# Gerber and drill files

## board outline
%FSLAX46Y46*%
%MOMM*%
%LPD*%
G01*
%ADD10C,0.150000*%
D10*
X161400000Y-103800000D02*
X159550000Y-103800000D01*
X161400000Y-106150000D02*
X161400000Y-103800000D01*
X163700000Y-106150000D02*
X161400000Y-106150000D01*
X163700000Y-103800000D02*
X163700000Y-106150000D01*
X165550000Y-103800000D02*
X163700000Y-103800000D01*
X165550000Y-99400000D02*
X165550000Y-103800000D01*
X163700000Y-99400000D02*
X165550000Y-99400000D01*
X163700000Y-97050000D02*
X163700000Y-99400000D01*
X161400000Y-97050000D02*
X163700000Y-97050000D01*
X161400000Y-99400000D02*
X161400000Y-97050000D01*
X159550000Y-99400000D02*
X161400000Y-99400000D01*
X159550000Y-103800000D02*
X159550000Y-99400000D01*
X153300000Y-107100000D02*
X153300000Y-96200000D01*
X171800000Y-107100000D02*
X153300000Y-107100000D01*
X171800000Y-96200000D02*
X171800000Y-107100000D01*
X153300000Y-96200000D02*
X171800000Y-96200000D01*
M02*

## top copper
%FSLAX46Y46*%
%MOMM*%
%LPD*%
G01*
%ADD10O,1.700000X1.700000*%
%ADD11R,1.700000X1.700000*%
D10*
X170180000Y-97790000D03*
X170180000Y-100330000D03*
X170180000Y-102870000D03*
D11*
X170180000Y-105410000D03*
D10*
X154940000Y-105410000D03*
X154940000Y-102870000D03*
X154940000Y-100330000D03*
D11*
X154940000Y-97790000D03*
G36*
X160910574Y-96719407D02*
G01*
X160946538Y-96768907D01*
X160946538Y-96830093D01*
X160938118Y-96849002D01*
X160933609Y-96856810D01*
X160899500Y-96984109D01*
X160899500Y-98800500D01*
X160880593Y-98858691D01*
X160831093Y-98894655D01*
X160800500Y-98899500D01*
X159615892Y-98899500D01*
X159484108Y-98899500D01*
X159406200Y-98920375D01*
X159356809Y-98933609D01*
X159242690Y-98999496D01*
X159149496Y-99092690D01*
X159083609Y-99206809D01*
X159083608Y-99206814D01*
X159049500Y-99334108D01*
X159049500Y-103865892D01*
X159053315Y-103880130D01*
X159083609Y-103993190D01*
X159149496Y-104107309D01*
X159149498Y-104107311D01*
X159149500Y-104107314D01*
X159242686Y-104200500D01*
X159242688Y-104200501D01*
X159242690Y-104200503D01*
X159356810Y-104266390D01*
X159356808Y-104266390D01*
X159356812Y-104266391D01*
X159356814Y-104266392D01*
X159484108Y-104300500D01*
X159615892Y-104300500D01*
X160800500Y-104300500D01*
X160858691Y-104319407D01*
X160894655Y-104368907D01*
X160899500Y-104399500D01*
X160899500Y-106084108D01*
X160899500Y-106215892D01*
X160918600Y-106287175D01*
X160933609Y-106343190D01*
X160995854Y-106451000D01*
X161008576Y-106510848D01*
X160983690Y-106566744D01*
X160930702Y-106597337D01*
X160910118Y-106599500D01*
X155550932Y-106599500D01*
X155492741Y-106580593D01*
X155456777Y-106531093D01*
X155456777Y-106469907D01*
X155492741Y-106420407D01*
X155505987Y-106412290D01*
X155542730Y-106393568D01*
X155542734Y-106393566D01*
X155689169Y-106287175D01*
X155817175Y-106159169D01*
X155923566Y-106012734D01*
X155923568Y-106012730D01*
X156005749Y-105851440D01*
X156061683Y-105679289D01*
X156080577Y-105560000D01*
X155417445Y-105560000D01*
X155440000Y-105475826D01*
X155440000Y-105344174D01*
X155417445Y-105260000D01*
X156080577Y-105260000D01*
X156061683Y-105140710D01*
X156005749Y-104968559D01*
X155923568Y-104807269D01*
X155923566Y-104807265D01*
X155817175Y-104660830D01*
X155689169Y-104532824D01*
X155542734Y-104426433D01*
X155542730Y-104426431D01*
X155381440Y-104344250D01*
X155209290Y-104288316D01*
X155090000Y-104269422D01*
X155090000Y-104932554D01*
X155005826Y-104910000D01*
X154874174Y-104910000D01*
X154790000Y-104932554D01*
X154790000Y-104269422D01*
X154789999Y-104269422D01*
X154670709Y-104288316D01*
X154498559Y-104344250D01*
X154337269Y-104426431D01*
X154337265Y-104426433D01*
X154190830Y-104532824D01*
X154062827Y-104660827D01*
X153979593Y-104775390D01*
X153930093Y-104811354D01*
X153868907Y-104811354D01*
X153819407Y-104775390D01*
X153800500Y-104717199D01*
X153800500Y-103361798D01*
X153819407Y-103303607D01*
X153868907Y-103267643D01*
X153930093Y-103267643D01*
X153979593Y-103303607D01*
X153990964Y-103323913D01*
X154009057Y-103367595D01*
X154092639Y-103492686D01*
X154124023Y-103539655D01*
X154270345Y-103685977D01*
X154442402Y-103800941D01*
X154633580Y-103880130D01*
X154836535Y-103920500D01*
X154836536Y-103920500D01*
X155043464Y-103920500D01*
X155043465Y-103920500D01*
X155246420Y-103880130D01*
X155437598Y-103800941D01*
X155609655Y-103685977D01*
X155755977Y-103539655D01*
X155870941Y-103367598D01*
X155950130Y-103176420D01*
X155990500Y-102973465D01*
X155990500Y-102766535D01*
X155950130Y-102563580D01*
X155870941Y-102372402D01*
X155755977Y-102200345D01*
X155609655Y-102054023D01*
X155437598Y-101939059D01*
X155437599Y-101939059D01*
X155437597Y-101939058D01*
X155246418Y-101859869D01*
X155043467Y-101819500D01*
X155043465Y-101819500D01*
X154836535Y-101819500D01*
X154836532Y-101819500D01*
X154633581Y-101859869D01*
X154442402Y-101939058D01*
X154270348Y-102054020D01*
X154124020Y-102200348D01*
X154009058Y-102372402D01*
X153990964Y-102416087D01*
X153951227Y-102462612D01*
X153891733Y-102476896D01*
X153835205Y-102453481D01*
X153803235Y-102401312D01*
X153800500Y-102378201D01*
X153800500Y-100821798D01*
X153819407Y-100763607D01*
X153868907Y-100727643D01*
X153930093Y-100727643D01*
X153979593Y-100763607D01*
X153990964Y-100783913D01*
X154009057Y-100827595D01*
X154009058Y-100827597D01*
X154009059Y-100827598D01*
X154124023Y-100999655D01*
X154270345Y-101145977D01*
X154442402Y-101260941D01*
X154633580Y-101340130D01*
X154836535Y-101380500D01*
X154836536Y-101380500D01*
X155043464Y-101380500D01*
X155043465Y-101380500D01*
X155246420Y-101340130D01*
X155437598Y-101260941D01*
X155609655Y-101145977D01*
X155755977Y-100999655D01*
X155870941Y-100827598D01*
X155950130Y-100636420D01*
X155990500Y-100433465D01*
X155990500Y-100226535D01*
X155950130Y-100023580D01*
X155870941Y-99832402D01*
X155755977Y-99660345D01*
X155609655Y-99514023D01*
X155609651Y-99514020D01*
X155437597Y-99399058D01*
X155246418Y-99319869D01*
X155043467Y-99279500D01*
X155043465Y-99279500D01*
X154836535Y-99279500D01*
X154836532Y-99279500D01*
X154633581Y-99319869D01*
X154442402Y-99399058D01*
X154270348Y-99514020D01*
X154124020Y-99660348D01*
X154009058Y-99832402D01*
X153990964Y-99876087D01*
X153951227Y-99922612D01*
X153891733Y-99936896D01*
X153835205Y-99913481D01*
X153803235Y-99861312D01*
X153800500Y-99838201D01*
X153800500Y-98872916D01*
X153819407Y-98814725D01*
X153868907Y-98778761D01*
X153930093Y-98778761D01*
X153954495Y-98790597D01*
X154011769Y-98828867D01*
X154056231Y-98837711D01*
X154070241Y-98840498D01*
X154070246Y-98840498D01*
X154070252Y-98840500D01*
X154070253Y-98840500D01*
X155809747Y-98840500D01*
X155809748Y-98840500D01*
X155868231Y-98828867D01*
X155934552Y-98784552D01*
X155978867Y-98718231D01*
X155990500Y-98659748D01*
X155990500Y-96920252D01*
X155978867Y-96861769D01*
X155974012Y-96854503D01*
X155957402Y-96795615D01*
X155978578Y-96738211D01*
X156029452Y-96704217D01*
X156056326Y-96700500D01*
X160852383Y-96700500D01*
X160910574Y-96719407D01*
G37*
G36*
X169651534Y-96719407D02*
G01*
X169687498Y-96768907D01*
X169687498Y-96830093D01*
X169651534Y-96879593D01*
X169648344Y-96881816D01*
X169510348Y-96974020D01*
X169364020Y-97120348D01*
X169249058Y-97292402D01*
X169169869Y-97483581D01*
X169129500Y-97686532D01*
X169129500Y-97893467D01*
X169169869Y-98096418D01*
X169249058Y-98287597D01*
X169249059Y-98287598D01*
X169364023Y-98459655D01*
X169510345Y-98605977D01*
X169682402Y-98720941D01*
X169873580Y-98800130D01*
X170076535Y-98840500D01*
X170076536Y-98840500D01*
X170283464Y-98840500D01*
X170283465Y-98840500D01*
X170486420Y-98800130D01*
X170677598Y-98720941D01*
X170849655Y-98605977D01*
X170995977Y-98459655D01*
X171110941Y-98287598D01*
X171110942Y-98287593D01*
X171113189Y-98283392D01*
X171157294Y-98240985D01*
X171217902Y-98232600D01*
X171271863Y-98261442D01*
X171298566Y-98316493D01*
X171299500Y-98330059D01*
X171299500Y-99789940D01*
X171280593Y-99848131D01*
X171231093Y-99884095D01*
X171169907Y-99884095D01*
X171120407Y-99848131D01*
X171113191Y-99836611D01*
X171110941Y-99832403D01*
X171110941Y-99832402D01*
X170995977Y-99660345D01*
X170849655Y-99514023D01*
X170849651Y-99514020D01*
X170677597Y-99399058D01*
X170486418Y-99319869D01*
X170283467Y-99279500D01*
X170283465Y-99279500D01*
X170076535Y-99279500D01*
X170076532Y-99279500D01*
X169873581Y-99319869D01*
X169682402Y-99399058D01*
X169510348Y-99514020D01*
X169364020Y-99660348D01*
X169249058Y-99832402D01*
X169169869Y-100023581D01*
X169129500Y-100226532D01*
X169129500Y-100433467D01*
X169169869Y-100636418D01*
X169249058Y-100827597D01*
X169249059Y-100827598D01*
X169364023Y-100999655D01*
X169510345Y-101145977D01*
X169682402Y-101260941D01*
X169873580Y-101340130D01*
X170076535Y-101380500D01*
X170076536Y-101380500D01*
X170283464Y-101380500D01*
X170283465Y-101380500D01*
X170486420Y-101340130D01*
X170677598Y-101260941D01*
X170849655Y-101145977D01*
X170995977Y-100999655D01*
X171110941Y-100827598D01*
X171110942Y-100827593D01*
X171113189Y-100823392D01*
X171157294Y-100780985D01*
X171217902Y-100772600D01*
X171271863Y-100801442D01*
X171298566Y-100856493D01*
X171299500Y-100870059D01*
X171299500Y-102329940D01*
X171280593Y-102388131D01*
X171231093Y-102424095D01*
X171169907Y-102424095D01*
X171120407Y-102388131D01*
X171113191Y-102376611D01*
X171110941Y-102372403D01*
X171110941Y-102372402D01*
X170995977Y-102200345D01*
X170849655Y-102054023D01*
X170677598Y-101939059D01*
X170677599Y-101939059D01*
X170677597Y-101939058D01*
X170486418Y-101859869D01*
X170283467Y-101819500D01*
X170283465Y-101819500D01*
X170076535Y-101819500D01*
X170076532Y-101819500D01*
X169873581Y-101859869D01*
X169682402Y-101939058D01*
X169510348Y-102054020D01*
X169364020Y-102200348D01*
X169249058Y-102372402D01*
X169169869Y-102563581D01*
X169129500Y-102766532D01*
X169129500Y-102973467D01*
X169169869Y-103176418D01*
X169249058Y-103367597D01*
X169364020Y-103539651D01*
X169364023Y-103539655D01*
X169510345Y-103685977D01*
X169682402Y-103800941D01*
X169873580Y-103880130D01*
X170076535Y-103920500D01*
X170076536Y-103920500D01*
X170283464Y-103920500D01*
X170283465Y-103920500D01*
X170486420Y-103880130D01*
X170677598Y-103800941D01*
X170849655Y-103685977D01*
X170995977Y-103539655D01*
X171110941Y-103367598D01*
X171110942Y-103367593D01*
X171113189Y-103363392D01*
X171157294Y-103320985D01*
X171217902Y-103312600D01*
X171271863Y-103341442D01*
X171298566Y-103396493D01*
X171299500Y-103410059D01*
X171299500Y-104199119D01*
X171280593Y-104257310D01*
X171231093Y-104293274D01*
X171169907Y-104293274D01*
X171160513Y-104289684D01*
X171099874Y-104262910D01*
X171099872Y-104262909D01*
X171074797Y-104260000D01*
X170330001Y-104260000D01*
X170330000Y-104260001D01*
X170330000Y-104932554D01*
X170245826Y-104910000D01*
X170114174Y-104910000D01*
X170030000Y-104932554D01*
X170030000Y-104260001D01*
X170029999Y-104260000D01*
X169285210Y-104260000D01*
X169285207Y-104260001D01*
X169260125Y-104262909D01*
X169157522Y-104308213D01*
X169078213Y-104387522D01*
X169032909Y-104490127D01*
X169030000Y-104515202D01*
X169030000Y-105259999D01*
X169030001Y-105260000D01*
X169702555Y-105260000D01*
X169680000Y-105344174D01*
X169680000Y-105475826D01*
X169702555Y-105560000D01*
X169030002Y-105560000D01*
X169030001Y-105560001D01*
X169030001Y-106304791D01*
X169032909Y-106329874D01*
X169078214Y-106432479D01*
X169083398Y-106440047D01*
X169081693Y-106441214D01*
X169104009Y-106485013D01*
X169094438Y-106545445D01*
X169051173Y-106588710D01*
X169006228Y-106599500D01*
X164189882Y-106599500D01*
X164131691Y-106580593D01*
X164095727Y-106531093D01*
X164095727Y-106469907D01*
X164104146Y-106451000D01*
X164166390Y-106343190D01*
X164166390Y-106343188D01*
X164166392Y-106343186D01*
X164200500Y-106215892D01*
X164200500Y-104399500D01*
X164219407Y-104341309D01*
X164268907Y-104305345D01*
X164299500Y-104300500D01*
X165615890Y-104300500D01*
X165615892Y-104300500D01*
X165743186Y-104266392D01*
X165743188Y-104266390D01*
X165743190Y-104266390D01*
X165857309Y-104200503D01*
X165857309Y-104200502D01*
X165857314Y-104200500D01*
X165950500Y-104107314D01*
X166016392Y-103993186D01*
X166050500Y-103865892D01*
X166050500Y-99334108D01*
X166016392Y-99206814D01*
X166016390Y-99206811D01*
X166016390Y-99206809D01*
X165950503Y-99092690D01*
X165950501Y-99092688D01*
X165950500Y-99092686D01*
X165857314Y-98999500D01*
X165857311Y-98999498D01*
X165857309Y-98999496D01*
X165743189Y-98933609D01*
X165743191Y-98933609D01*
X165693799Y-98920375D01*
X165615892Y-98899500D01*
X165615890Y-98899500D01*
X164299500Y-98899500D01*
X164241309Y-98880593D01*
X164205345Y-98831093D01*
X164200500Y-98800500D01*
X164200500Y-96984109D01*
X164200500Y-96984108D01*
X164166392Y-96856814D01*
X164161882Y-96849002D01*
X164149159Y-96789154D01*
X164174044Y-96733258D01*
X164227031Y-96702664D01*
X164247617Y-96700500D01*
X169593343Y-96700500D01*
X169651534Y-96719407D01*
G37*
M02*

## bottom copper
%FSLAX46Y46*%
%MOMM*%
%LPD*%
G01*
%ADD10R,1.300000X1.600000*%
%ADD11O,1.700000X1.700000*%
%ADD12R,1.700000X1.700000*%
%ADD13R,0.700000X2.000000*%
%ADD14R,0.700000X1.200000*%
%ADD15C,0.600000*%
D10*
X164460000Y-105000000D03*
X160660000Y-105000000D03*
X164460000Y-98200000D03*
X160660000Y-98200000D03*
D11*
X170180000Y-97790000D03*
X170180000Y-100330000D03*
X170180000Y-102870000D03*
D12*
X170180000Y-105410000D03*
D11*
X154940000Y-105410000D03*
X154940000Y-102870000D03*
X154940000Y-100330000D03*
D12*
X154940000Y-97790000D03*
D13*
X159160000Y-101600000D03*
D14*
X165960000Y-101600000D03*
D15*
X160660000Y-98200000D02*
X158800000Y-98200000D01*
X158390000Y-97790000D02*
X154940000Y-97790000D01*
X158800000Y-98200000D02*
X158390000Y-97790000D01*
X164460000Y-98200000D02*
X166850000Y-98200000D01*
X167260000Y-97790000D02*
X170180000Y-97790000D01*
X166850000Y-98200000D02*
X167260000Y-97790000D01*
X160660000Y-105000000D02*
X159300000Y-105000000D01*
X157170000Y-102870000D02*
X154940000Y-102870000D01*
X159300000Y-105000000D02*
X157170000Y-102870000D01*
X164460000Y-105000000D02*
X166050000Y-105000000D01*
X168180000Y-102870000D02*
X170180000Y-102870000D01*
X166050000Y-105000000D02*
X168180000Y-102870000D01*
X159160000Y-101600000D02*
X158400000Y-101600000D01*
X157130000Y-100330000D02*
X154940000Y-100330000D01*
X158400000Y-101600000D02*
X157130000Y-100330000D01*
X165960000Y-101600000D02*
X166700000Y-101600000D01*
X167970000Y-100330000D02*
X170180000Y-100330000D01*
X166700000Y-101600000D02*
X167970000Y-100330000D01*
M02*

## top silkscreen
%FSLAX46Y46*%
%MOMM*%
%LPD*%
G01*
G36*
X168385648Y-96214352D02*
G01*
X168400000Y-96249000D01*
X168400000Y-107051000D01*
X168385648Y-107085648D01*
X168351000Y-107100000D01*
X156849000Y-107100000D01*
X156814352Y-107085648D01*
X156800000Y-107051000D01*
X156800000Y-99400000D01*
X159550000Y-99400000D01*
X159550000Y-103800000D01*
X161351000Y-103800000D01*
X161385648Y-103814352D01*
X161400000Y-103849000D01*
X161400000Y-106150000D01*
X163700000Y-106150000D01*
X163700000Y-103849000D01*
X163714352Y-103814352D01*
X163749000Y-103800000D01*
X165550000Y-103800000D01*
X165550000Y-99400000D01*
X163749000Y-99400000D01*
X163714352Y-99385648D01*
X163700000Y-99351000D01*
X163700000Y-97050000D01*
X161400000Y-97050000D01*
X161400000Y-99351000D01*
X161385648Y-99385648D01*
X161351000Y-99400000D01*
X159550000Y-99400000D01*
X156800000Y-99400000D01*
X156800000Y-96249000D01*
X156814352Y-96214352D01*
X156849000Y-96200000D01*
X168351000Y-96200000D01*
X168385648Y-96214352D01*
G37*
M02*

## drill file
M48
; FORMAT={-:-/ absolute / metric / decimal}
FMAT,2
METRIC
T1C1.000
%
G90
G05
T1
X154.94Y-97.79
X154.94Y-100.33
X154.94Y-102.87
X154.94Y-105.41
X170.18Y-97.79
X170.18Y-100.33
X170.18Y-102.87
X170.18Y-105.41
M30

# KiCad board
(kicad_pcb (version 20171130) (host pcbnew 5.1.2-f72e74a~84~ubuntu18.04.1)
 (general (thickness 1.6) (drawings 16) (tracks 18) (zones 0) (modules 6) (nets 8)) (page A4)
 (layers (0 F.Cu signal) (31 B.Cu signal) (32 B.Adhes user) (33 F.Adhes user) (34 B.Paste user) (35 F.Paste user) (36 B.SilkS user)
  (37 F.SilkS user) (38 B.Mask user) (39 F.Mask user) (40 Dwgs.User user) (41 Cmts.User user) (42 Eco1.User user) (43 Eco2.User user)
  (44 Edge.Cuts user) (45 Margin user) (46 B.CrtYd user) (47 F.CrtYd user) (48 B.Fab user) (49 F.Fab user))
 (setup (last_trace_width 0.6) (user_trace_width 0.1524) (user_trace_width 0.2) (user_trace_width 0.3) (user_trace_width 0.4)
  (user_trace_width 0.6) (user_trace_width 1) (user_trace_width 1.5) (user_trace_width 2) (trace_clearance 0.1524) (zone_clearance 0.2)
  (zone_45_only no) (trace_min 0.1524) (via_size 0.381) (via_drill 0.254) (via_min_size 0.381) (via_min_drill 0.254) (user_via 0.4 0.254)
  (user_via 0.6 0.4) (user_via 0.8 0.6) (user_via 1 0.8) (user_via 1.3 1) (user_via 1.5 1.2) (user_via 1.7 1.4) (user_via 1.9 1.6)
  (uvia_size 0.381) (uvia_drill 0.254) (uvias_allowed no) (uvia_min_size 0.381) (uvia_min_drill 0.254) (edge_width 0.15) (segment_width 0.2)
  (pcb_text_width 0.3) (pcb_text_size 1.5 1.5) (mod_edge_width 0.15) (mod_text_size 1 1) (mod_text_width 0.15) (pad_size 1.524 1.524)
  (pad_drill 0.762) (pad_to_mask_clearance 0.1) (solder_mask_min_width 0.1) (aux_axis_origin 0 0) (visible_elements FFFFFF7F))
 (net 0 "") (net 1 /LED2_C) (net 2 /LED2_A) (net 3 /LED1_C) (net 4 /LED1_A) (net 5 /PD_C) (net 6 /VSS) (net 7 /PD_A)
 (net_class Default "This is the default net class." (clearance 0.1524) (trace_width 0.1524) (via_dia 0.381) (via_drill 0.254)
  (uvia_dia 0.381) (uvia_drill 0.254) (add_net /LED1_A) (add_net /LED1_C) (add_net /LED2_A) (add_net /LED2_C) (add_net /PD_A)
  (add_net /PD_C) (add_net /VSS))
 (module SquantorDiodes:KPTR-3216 (layer B.Cu) (at 162.56 105 180)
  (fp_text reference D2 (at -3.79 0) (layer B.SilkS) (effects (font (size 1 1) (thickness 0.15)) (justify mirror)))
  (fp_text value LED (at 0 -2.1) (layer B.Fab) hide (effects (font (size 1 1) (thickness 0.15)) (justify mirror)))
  (pad 1 smd rect (at -1.9 0 180) (size 1.3 1.6) (layers B.Cu B.Paste B.Mask) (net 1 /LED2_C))
  (pad 2 smd rect (at 1.9 0 180) (size 1.3 1.6) (layers B.Cu B.Paste B.Mask) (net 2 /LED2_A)))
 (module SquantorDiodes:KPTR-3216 (layer B.Cu) (at 162.56 98.2 180)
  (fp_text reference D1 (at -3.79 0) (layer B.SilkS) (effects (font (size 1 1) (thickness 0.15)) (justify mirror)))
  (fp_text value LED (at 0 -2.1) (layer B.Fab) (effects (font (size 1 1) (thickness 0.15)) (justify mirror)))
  (pad 1 smd rect (at -1.9 0 180) (size 1.3 1.6) (layers B.Cu B.Paste B.Mask) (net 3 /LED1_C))
  (pad 2 smd rect (at 1.9 0 180) (size 1.3 1.6) (layers B.Cu B.Paste B.Mask) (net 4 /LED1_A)))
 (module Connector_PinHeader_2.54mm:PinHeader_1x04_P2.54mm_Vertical (layer B.Cu) (at 170.18 105.41)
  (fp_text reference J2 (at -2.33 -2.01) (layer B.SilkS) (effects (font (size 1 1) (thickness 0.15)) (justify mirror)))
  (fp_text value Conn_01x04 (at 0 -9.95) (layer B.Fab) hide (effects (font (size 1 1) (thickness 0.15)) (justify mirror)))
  (pad 4 thru_hole oval (at 0 -7.62) (size 1.7 1.7) (drill 1) (layers *.Cu *.Mask) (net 3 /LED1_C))
  (pad 3 thru_hole oval (at 0 -5.08) (size 1.7 1.7) (drill 1) (layers *.Cu *.Mask) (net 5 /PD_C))
  (pad 2 thru_hole oval (at 0 -2.54) (size 1.7 1.7) (drill 1) (layers *.Cu *.Mask) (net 1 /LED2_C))
  (pad 1 thru_hole rect (at 0 0) (size 1.7 1.7) (drill 1) (layers *.Cu *.Mask) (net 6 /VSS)))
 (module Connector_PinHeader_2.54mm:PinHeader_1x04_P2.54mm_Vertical (layer B.Cu) (at 154.94 97.79 180)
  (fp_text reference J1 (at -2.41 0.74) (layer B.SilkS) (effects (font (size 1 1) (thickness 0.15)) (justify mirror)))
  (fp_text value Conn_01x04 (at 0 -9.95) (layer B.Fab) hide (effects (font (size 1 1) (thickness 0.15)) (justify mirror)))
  (pad 4 thru_hole oval (at 0 -7.62 180) (size 1.7 1.7) (drill 1) (layers *.Cu *.Mask) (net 6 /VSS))
  (pad 3 thru_hole oval (at 0 -5.08 180) (size 1.7 1.7) (drill 1) (layers *.Cu *.Mask) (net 2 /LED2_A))
  (pad 2 thru_hole oval (at 0 -2.54 180) (size 1.7 1.7) (drill 1) (layers *.Cu *.Mask) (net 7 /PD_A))
  (pad 1 thru_hole rect (at 0 0 180) (size 1.7 1.7) (drill 1) (layers *.Cu *.Mask) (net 4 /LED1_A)))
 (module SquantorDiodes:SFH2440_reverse (layer B.Cu) (at 162.56 101.6 180)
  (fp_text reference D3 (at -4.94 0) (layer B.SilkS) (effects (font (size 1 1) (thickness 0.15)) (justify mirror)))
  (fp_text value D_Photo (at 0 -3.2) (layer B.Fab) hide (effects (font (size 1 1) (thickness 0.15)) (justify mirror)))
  (pad 2 smd rect (at 3.4 0 180) (size 0.7 2) (layers B.Cu B.Paste B.Mask) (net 7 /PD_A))
  (pad 1 smd rect (at -3.4 0 180) (size 0.7 1.2) (layers B.Cu B.Paste B.Mask) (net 5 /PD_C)))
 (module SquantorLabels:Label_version (layer B.Cu) (at 157.25 102.6 90)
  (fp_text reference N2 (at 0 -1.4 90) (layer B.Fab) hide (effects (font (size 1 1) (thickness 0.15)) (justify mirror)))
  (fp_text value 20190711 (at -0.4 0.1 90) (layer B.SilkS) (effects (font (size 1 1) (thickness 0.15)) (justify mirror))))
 (gr_line (start 161.4 103.8) (end 159.55 103.8) (layer Edge.Cuts) (width 0.15))
 (gr_line (start 161.4 106.15) (end 161.4 103.8) (layer Edge.Cuts) (width 0.15))
 (gr_line (start 163.7 106.15) (end 161.4 106.15) (layer Edge.Cuts) (width 0.15))
 (gr_line (start 163.7 103.8) (end 163.7 106.15) (layer Edge.Cuts) (width 0.15))
 (gr_line (start 165.55 103.8) (end 163.7 103.8) (layer Edge.Cuts) (width 0.15))
 (gr_line (start 165.55 99.4) (end 165.55 103.8) (layer Edge.Cuts) (width 0.15))
 (gr_line (start 163.7 99.4) (end 165.55 99.4) (layer Edge.Cuts) (width 0.15))
 (gr_line (start 163.7 97.05) (end 163.7 99.4) (layer Edge.Cuts) (width 0.15))
 (gr_line (start 161.4 97.05) (end 163.7 97.05) (layer Edge.Cuts) (width 0.15))
 (gr_line (start 161.4 99.4) (end 161.4 97.05) (layer Edge.Cuts) (width 0.15))
 (gr_line (start 159.55 99.4) (end 161.4 99.4) (layer Edge.Cuts) (width 0.15))
 (gr_line (start 159.55 103.8) (end 159.55 99.4) (layer Edge.Cuts) (width 0.15))
 (gr_line (start 153.3 107.1) (end 153.3 96.2) (layer Edge.Cuts) (width 0.15))
 (gr_line (start 171.8 107.1) (end 153.3 107.1) (layer Edge.Cuts) (width 0.15))
 (gr_line (start 171.8 96.2) (end 171.8 107.1) (layer Edge.Cuts) (width 0.15))
 (gr_line (start 153.3 96.2) (end 171.8 96.2) (layer Edge.Cuts) (width 0.15))
 (segment (start 160.66 98.2) (end 158.8 98.2) (width 0.6) (layer B.Cu) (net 4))
 (segment (start 158.39 97.79) (end 154.94 97.79) (width 0.6) (layer B.Cu) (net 4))
 (segment (start 158.8 98.2) (end 158.39 97.79) (width 0.6) (layer B.Cu) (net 4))
 (segment (start 164.46 98.2) (end 166.85 98.2) (width 0.6) (layer B.Cu) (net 3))
 (segment (start 167.26 97.79) (end 170.18 97.79) (width 0.6) (layer B.Cu) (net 3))
 (segment (start 166.85 98.2) (end 167.26 97.79) (width 0.6) (layer B.Cu) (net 3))
 (segment (start 160.66 105) (end 159.3 105) (width 0.6) (layer B.Cu) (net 2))
 (segment (start 157.17 102.87) (end 154.94 102.87) (width 0.6) (layer B.Cu) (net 2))
 (segment (start 159.3 105) (end 157.17 102.87) (width 0.6) (layer B.Cu) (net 2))
 (segment (start 164.46 105) (end 166.05 105) (width 0.6) (layer B.Cu) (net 1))
 (segment (start 168.18 102.87) (end 170.18 102.87) (width 0.6) (layer B.Cu) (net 1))
 (segment (start 166.05 105) (end 168.18 102.87) (width 0.6) (layer B.Cu) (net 1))
 (segment (start 159.16 101.6) (end 158.4 101.6) (width 0.6) (layer B.Cu) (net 7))
 (segment (start 157.13 100.33) (end 154.94 100.33) (width 0.6) (layer B.Cu) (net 7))
 (segment (start 158.4 101.6) (end 157.13 100.33) (width 0.6) (layer B.Cu) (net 7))
 (segment (start 165.96 101.6) (end 166.7 101.6) (width 0.6) (layer B.Cu) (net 5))
 (segment (start 167.97 100.33) (end 170.18 100.33) (width 0.6) (layer B.Cu) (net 5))
 (segment (start 166.7 101.6) (end 167.97 100.33) (width 0.6) (layer B.Cu) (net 5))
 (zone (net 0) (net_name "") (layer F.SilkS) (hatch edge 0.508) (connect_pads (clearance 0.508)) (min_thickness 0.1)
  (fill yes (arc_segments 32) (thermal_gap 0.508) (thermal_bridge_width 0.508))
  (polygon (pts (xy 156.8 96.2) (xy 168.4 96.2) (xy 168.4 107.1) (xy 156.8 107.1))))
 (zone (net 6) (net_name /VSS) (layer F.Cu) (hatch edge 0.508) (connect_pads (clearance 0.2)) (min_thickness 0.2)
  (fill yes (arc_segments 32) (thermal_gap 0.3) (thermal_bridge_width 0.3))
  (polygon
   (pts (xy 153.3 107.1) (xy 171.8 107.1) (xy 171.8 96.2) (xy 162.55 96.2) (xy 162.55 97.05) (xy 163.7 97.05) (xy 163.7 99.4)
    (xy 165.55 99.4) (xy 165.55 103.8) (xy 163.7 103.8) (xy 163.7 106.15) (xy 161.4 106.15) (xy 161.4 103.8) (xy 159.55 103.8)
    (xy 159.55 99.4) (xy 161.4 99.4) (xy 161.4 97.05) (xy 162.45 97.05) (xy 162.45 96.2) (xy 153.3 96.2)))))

